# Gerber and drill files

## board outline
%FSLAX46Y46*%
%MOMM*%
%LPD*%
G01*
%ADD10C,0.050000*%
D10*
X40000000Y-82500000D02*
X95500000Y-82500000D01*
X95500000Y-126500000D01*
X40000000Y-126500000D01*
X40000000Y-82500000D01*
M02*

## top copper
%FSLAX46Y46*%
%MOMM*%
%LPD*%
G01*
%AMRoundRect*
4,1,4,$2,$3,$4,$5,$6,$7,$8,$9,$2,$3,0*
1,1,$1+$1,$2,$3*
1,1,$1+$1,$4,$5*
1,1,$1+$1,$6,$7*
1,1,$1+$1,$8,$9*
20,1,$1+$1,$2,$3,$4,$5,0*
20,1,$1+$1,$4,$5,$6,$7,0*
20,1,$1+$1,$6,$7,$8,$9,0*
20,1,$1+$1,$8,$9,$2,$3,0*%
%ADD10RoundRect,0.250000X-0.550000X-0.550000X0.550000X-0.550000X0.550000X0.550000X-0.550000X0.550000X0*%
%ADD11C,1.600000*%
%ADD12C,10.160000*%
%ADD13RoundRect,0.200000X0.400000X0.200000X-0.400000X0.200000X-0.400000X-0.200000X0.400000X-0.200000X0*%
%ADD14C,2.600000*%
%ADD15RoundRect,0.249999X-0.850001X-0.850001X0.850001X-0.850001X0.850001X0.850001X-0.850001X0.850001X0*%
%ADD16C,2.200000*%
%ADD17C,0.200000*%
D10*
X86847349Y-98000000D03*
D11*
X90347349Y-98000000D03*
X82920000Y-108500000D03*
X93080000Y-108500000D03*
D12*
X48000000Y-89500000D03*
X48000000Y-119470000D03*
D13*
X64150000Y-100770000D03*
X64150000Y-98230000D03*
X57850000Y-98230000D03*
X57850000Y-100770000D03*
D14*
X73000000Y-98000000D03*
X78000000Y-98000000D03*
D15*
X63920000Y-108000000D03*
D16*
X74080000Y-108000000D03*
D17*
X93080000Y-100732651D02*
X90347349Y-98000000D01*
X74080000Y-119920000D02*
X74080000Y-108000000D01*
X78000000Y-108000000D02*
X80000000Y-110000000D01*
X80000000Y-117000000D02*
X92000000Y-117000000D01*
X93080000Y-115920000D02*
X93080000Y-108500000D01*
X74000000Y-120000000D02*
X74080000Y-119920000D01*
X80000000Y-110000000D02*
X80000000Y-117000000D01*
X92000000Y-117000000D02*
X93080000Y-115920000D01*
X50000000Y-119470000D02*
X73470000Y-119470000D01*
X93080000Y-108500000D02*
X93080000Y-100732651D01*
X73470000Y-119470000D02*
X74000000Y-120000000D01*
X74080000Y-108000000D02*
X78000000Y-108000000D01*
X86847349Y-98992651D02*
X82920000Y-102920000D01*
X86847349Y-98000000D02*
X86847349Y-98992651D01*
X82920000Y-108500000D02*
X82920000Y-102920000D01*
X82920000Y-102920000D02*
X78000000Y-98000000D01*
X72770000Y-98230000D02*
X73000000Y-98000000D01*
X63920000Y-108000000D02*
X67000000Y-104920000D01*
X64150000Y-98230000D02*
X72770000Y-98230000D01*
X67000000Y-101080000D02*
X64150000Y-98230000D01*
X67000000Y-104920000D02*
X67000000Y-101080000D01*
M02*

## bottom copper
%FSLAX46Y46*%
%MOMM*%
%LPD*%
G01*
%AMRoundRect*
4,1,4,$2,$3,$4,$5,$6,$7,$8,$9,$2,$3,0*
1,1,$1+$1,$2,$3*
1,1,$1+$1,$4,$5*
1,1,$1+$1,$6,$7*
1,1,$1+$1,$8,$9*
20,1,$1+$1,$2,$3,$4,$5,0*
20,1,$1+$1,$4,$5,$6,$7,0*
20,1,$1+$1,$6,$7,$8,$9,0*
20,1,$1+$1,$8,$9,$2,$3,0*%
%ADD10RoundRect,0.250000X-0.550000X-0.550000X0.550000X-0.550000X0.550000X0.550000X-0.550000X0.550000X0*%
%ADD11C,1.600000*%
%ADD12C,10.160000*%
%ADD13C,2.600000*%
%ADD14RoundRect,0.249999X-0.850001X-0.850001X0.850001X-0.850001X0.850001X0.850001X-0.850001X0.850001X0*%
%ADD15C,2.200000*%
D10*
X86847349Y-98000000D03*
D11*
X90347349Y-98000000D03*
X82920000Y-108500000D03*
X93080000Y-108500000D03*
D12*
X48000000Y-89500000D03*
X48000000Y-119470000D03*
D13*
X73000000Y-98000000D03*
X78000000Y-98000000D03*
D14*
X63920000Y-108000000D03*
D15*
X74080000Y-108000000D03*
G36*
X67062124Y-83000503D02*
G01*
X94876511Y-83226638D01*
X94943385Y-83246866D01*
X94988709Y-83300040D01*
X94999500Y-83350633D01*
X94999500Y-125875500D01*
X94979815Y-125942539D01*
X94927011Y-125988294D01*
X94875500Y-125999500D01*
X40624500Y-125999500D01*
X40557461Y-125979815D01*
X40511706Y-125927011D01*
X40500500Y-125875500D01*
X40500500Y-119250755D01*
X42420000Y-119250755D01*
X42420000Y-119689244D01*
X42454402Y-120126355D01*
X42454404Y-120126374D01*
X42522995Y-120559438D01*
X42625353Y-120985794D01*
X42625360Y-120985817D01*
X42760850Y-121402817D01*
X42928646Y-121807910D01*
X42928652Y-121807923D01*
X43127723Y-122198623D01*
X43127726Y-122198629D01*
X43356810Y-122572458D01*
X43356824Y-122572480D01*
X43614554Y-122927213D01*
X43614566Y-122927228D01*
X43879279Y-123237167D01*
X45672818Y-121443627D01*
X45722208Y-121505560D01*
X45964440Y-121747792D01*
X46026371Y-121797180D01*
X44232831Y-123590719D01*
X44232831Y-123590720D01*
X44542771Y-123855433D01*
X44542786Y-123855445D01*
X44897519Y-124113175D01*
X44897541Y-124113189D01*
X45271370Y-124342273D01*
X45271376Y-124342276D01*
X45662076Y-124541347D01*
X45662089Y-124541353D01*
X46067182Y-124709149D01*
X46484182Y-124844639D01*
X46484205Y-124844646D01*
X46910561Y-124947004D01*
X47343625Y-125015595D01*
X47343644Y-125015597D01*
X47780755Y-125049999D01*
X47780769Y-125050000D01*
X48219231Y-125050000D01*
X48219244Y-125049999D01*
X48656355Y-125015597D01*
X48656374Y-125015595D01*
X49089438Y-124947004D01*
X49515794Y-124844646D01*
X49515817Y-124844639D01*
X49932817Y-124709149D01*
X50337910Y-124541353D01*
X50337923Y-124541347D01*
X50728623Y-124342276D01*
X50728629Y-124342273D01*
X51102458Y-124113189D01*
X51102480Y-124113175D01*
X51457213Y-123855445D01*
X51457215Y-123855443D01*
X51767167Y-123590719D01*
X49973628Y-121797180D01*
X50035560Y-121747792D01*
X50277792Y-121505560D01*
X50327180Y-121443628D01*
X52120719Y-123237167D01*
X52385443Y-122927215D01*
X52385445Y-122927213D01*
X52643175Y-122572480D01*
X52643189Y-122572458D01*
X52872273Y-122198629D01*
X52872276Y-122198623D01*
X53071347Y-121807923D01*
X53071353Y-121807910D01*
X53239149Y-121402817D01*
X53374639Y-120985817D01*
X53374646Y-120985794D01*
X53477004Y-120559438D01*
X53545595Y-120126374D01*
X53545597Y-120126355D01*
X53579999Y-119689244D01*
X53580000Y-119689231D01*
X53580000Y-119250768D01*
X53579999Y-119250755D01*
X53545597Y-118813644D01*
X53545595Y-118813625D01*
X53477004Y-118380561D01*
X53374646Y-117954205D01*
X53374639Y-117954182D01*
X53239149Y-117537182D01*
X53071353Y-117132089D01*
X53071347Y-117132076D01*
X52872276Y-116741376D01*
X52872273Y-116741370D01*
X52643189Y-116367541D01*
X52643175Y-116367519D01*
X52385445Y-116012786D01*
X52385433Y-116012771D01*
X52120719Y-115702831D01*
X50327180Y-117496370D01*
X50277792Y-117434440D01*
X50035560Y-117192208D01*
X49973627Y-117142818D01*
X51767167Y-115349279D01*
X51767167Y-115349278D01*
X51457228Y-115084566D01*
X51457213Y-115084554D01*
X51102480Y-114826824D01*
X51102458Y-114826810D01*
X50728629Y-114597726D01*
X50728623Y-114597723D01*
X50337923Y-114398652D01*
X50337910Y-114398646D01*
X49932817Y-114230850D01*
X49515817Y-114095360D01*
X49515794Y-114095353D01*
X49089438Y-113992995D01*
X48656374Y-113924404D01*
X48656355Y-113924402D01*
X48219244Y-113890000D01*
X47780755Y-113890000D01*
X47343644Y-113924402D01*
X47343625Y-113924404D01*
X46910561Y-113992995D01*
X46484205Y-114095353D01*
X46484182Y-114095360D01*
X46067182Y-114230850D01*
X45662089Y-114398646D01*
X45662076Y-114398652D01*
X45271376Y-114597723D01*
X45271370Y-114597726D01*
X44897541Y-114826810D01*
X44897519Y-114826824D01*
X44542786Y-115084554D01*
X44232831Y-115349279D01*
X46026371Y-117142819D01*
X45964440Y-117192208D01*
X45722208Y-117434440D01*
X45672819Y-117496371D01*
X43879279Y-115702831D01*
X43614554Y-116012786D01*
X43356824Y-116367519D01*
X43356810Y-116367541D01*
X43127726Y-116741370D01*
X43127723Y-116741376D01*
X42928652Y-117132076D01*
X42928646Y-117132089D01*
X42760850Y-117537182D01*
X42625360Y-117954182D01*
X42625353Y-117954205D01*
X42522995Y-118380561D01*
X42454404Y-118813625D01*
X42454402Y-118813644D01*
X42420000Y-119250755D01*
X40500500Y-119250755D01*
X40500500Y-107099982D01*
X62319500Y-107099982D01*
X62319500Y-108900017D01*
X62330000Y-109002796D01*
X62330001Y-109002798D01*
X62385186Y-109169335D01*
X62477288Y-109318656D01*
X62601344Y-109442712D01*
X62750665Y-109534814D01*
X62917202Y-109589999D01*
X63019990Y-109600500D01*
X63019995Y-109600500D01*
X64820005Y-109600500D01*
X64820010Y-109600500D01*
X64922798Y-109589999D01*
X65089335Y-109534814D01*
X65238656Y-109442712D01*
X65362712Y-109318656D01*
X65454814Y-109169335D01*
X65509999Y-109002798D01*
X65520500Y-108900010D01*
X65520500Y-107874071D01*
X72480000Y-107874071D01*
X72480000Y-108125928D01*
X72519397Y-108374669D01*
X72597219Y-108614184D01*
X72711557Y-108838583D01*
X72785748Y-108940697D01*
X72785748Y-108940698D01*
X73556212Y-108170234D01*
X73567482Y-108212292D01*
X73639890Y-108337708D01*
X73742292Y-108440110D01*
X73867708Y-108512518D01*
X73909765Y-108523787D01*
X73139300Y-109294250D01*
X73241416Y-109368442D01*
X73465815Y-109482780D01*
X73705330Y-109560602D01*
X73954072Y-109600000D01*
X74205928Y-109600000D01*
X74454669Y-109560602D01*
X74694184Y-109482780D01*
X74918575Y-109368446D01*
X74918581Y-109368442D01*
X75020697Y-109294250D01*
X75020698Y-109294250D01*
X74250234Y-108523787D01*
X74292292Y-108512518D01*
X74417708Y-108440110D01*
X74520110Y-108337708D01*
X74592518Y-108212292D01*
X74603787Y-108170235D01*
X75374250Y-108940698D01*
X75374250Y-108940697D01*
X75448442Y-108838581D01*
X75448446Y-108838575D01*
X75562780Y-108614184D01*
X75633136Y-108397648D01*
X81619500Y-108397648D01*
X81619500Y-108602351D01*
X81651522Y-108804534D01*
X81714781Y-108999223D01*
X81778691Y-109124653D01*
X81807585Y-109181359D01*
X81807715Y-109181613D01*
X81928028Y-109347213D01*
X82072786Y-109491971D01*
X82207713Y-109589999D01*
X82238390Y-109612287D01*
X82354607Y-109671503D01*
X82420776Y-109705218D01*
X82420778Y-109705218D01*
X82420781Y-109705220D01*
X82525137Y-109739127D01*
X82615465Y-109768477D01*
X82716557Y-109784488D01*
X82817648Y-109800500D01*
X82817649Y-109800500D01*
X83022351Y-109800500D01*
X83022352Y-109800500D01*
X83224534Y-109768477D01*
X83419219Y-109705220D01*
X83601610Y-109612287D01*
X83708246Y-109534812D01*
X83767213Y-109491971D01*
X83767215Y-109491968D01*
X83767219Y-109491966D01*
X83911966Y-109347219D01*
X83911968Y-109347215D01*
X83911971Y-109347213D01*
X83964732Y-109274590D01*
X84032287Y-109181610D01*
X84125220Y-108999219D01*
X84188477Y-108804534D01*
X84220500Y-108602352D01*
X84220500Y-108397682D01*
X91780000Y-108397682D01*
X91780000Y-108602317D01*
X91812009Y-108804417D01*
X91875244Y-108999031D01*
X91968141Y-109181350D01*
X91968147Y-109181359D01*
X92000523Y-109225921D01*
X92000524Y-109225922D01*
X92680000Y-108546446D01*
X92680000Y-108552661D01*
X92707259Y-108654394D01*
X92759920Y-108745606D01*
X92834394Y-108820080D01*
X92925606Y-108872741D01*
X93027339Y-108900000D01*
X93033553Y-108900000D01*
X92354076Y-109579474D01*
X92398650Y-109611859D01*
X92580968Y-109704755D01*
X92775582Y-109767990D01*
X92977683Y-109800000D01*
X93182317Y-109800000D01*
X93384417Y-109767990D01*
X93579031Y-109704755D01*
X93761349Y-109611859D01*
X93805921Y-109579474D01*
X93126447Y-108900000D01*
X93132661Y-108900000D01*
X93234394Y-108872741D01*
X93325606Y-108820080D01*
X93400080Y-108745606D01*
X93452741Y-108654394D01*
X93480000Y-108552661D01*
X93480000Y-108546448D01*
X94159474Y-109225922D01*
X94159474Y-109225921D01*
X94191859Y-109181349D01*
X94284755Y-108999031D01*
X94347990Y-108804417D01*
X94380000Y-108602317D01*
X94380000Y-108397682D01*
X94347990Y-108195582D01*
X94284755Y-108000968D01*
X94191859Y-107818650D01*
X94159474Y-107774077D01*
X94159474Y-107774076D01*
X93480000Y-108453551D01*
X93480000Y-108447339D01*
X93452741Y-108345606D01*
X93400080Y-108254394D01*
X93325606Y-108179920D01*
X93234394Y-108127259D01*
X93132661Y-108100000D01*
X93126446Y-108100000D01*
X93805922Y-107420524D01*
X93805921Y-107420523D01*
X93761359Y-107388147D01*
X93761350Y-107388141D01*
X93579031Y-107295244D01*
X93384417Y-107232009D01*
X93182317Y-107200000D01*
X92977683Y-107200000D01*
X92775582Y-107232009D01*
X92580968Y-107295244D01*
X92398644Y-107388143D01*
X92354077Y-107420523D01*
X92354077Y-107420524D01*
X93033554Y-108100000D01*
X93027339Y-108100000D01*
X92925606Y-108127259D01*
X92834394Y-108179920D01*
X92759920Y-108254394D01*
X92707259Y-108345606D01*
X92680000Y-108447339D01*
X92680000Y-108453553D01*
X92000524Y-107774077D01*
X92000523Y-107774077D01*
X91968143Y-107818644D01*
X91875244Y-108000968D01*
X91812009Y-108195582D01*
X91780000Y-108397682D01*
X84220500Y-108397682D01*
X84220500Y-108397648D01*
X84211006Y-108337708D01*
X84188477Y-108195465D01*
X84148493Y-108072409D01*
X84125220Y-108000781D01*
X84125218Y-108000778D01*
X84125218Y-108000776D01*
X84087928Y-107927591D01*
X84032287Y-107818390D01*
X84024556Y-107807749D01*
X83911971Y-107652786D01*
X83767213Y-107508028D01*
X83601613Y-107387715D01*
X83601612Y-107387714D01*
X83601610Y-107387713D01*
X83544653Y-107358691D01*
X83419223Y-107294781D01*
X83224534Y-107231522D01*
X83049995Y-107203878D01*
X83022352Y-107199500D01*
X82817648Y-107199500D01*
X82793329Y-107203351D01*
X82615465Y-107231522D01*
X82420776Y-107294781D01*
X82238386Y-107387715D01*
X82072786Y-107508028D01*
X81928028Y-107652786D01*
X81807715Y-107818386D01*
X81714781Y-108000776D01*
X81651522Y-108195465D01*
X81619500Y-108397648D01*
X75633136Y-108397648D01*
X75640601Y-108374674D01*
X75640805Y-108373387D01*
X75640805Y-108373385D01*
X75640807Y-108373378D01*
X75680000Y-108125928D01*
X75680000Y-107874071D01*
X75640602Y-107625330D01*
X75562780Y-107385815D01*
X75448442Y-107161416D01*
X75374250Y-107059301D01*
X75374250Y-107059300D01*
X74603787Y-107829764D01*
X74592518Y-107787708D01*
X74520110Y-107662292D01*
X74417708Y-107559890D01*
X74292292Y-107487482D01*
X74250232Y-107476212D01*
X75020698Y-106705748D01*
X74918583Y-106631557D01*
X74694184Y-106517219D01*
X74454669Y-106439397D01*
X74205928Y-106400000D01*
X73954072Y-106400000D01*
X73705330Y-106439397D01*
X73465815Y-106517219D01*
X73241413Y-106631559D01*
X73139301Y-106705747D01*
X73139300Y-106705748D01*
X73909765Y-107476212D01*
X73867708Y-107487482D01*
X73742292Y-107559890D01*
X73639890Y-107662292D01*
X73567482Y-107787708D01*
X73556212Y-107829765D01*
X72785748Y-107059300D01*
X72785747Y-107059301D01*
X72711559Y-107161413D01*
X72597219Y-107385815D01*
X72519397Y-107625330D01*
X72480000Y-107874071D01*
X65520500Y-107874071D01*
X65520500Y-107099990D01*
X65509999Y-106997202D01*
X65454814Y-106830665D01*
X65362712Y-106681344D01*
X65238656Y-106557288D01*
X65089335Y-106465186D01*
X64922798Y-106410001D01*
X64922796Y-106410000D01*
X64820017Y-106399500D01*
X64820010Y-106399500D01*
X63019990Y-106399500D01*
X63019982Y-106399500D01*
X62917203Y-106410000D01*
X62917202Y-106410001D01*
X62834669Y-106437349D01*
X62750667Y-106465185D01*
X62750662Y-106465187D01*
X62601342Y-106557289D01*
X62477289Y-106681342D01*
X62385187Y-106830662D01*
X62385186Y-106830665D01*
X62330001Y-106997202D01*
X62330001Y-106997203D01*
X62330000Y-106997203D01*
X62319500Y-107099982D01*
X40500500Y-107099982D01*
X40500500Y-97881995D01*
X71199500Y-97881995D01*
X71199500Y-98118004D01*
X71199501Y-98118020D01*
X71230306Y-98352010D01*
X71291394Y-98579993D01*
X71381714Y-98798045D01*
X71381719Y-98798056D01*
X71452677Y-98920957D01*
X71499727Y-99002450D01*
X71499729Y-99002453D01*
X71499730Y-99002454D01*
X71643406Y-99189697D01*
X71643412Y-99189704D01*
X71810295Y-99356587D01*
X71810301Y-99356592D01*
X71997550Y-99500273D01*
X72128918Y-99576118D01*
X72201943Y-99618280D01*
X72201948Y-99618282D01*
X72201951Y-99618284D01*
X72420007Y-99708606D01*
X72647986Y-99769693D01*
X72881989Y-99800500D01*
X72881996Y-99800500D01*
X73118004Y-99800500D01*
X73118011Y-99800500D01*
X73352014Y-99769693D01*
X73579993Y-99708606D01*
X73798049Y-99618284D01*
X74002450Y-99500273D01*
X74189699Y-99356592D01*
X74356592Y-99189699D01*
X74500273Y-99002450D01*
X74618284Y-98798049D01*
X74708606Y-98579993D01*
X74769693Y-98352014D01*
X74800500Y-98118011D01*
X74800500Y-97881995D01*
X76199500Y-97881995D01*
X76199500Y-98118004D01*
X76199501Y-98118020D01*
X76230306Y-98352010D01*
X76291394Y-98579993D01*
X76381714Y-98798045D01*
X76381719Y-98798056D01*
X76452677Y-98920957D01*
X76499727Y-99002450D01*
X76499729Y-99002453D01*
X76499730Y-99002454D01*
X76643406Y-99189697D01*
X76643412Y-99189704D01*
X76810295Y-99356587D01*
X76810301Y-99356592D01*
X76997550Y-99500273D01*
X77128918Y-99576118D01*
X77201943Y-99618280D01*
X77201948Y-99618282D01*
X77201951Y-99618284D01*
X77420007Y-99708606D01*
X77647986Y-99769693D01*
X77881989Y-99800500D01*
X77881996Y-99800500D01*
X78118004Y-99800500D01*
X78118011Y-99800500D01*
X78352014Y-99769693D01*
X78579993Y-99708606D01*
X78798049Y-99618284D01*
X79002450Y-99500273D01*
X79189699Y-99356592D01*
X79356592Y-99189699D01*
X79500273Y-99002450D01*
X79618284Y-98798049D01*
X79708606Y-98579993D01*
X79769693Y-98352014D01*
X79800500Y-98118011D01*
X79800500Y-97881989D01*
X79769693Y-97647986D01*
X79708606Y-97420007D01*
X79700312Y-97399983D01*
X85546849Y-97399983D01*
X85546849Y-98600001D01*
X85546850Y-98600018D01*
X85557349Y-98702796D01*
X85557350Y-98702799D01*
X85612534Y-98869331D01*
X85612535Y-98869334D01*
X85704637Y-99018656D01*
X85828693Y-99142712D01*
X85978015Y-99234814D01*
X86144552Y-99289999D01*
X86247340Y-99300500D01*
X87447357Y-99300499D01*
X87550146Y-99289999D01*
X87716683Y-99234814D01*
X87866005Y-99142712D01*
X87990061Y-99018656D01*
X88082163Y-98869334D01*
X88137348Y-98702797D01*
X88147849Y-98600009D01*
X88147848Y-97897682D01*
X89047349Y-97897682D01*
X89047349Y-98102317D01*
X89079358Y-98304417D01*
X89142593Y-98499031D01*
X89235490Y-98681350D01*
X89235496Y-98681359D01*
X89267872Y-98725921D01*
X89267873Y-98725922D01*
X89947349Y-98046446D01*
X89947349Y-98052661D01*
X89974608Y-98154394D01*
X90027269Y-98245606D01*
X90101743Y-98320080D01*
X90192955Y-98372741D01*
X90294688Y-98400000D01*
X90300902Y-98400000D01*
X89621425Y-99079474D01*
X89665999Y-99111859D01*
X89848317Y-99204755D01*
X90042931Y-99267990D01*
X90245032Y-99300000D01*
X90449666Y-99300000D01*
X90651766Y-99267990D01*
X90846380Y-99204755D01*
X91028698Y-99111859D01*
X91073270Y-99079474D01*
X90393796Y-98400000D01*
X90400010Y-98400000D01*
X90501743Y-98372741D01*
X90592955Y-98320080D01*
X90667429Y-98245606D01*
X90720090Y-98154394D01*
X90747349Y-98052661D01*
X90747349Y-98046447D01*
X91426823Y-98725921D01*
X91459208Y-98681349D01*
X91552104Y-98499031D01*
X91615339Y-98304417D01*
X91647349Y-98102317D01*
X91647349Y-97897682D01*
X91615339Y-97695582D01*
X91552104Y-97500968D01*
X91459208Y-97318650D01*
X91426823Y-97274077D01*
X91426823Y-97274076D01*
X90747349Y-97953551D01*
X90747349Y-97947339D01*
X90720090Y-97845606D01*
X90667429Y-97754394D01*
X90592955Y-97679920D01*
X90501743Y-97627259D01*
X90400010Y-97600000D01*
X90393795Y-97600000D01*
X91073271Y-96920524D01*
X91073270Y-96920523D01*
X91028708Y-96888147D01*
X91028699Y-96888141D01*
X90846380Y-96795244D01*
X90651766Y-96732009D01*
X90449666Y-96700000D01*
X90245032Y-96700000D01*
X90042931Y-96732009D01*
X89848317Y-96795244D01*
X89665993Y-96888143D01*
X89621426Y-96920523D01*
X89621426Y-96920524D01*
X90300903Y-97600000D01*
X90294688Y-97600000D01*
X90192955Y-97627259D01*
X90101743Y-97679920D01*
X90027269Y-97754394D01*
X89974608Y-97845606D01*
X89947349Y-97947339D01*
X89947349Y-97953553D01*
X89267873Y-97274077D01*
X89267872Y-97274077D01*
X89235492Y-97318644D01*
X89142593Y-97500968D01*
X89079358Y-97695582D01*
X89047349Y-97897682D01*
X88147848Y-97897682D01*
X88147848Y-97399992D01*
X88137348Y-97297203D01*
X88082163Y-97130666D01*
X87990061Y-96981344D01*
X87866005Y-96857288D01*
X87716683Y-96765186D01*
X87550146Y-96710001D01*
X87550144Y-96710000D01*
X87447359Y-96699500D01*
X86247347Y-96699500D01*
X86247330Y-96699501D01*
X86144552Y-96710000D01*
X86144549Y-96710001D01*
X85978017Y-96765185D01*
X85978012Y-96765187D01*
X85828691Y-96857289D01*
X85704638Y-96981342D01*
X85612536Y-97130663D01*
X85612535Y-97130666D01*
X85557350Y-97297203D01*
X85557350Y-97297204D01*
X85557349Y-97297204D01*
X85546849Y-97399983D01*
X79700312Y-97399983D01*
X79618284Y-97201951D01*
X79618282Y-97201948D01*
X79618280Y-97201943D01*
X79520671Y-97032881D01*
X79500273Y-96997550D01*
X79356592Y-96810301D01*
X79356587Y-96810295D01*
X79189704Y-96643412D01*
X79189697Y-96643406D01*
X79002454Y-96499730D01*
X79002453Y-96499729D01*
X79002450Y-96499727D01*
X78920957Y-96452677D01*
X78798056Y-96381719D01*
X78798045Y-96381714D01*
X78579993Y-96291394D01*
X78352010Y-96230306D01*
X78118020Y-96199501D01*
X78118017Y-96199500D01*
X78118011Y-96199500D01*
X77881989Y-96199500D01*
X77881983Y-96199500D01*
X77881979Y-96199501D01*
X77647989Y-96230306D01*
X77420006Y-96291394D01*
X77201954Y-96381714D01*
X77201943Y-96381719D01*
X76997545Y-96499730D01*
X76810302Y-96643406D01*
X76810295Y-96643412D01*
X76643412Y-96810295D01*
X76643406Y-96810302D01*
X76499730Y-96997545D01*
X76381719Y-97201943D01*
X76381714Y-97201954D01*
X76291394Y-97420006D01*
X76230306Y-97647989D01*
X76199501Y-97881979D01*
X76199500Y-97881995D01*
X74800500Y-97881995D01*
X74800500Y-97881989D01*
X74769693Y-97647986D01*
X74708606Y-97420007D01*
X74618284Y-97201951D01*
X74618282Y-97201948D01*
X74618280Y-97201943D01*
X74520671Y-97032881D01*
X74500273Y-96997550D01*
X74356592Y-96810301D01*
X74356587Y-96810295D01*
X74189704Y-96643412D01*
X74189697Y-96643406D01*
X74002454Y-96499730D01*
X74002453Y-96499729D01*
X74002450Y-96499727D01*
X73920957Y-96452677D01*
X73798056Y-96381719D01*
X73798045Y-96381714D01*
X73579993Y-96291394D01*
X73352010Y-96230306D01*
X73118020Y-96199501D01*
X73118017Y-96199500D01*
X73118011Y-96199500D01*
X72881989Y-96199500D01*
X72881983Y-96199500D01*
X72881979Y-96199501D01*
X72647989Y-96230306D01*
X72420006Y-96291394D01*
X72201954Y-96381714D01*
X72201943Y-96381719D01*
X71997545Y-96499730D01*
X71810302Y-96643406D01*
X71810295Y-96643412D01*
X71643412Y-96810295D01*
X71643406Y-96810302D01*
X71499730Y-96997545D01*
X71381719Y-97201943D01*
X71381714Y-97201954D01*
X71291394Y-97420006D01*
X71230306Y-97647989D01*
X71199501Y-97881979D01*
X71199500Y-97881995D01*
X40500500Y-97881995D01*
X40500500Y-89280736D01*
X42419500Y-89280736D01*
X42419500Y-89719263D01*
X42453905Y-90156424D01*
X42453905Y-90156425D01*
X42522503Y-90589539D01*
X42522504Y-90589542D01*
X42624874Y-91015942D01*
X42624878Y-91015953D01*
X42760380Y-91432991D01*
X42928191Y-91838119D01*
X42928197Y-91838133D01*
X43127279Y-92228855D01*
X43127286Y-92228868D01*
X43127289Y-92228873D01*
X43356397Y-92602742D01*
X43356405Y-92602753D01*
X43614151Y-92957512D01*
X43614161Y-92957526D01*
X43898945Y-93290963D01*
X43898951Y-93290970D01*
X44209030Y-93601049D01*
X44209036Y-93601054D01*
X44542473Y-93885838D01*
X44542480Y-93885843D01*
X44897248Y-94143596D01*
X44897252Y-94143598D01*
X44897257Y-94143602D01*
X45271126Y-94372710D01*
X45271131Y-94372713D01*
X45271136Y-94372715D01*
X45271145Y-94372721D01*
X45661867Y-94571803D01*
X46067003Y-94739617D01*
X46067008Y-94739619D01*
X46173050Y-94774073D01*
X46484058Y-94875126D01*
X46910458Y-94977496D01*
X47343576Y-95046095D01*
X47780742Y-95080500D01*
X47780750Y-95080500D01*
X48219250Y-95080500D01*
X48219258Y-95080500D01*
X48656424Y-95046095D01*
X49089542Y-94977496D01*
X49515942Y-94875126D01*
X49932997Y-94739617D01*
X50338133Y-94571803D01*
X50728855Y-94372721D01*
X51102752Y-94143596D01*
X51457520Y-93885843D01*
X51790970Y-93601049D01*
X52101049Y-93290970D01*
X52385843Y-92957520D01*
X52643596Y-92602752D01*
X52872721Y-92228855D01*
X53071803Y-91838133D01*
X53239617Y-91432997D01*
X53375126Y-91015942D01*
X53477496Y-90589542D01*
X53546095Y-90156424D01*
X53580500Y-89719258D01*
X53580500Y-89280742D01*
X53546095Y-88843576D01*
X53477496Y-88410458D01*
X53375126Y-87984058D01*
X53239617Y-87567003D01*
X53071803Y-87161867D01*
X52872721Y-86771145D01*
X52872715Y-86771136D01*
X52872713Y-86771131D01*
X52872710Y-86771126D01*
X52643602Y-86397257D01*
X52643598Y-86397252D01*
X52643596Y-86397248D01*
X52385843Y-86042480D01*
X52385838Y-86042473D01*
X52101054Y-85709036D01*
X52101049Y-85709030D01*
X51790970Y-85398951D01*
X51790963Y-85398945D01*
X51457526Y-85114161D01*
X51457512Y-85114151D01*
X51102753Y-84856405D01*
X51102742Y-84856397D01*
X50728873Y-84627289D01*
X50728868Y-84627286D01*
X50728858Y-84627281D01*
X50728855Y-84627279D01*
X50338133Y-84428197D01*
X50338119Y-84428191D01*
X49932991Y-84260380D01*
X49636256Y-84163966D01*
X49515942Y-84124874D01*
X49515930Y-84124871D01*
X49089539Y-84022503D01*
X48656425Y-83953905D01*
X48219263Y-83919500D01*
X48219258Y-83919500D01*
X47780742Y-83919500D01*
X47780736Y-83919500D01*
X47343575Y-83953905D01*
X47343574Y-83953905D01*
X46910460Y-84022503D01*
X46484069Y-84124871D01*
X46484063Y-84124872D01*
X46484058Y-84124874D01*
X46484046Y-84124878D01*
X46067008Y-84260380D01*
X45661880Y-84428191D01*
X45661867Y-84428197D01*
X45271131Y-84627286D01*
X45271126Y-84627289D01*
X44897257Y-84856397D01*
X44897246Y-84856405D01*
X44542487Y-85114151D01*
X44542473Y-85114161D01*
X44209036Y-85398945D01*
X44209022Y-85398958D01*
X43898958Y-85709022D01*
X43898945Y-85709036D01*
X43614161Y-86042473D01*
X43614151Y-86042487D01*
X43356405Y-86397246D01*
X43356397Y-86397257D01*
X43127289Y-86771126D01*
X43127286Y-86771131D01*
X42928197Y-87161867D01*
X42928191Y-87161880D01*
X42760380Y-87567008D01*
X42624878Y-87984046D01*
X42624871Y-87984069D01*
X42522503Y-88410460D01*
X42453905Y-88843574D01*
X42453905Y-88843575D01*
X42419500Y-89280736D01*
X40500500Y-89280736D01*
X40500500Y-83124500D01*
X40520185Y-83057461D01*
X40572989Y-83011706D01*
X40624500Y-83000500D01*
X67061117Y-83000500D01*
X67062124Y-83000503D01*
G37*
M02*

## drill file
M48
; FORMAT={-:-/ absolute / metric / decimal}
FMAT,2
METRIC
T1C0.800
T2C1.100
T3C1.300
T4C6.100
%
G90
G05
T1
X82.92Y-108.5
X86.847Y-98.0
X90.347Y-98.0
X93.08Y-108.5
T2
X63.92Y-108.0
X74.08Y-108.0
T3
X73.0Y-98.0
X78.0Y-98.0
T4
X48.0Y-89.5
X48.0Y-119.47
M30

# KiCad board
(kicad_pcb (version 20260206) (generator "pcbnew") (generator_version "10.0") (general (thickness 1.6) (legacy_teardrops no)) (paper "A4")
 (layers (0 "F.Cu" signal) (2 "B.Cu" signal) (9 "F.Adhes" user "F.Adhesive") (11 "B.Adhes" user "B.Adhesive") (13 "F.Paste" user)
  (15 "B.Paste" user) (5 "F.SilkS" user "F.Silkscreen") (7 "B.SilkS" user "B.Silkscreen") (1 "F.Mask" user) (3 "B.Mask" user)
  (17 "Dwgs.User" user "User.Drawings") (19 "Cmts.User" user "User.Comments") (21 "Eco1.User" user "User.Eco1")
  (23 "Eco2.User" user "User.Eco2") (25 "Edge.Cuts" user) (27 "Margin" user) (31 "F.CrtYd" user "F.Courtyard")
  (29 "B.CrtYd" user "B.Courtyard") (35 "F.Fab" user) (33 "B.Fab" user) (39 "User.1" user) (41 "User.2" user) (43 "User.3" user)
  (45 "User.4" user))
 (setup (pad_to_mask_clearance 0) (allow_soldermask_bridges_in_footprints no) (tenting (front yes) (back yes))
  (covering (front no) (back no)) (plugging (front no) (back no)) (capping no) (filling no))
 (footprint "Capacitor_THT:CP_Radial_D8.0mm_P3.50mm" (layer "F.Cu") (at 86.847349 98)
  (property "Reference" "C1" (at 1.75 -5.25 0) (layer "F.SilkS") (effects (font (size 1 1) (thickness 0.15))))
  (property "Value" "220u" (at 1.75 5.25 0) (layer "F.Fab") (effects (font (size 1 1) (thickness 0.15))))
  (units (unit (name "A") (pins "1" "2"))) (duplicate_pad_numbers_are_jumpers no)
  (pad "1" thru_hole roundrect (at 0 0) (size 1.6 1.6) (drill 0.8) (layers "*.Cu" "*.Mask") (remove_unused_layers no)
   (roundrect_rratio 0.15625) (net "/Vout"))
  (pad "2" thru_hole circle (at 3.5 0) (size 1.6 1.6) (drill 0.8) (layers "*.Cu" "*.Mask") (remove_unused_layers no) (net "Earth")))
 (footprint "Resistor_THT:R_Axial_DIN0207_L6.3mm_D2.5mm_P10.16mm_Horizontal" (layer "F.Cu") (at 82.92 108.5)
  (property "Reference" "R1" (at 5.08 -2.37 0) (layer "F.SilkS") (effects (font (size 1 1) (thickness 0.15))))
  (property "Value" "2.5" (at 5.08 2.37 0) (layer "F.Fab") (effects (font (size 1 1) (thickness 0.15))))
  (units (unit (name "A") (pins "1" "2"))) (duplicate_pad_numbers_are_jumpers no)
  (pad "1" thru_hole circle (at 0 0) (size 1.6 1.6) (drill 0.8) (layers "*.Cu" "*.Mask") (remove_unused_layers no) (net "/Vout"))
  (pad "2" thru_hole circle (at 10.16 0) (size 1.6 1.6) (drill 0.8) (layers "*.Cu" "*.Mask") (remove_unused_layers no) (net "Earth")))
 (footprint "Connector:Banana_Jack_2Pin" (layer "F.Cu") (at 48 89.5 -90)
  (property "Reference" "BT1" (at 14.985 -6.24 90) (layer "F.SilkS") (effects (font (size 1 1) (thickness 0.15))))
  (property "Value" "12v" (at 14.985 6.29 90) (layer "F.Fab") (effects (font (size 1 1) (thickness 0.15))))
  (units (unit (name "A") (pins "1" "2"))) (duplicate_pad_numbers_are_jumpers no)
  (pad "1" thru_hole circle (at 0 0 270) (size 10.16 10.16) (drill 6.1) (layers "*.Cu" "*.Mask") (remove_unused_layers no) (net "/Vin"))
  (pad "2" thru_hole circle (at 29.97 0 270) (size 10.16 10.16) (drill 6.1) (layers "*.Cu" "*.Mask") (remove_unused_layers no) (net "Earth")))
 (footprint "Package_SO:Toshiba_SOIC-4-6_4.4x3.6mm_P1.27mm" (layer "F.Cu") (at 61 99.5 180)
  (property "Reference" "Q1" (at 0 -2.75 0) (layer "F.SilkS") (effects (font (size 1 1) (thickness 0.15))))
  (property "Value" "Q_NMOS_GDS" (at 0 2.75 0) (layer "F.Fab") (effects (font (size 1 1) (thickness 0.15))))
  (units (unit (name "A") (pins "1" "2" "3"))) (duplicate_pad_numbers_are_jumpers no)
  (pad "1" smd roundrect (at -3.15 -1.27 180) (size 1.2 0.8) (layers "F.Cu" "F.Mask" "F.Paste") (roundrect_rratio 0.25)
   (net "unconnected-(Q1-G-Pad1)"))
  (pad "3" smd roundrect (at -3.15 1.27 180) (size 1.2 0.8) (layers "F.Cu" "F.Mask" "F.Paste") (roundrect_rratio 0.25) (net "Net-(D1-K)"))
  (pad "4" smd roundrect (at 3.15 1.27 180) (size 1.2 0.8) (layers "F.Cu" "F.Mask" "F.Paste") (roundrect_rratio 0.25))
  (pad "6" smd roundrect (at 3.15 -1.27 180) (size 1.2 0.8) (layers "F.Cu" "F.Mask" "F.Paste") (roundrect_rratio 0.25)))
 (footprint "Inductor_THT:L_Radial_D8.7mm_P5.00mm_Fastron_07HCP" (layer "F.Cu") (at 73 98)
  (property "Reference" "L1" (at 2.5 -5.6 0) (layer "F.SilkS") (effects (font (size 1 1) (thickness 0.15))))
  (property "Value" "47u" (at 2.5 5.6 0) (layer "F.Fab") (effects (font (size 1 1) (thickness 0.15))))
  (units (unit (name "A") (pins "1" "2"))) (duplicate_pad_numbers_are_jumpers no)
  (pad "1" thru_hole circle (at 0 0) (size 2.6 2.6) (drill 1.3) (layers "*.Cu" "*.Mask") (remove_unused_layers no) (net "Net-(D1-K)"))
  (pad "2" thru_hole circle (at 5 0) (size 2.6 2.6) (drill 1.3) (layers "*.Cu" "*.Mask") (remove_unused_layers no) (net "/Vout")))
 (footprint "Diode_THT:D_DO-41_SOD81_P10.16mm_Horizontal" (layer "F.Cu") (at 63.92 108)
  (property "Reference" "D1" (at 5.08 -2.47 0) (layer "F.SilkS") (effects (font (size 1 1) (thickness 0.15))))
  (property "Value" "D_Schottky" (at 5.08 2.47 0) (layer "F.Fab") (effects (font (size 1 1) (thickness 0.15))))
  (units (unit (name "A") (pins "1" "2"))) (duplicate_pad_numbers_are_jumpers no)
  (pad "1" thru_hole roundrect (at 0 0) (size 2.2 2.2) (drill 1.1) (layers "*.Cu" "*.Mask") (remove_unused_layers no)
   (roundrect_rratio 0.113636) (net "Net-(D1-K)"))
  (pad "2" thru_hole circle (at 10.16 0) (size 2.2 2.2) (drill 1.1) (layers "*.Cu" "*.Mask") (remove_unused_layers no) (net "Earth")))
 (gr_rect (start 40 82.5) (end 95.5 126.5) (stroke (width 0.05) (type default)) (fill no) (layer "Edge.Cuts"))
 (segment (start 93.08 100.732651) (end 90.347349 98) (width 0.2) (layer "F.Cu") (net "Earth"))
 (segment (start 74.08 119.92) (end 74.08 108) (width 0.2) (layer "F.Cu") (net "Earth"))
 (segment (start 78 108) (end 80 110) (width 0.2) (layer "F.Cu") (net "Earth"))
 (segment (start 80 117) (end 92 117) (width 0.2) (layer "F.Cu") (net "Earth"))
 (segment (start 93.08 115.92) (end 93.08 108.5) (width 0.2) (layer "F.Cu") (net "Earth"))
 (segment (start 74 120) (end 74.08 119.92) (width 0.2) (layer "F.Cu") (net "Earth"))
 (segment (start 80 110) (end 80 117) (width 0.2) (layer "F.Cu") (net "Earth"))
 (segment (start 92 117) (end 93.08 115.92) (width 0.2) (layer "F.Cu") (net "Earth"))
 (segment (start 50 119.47) (end 73.47 119.47) (width 0.2) (layer "F.Cu") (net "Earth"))
 (segment (start 93.08 108.5) (end 93.08 100.732651) (width 0.2) (layer "F.Cu") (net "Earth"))
 (segment (start 73.47 119.47) (end 74 120) (width 0.2) (layer "F.Cu") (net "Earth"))
 (segment (start 74.08 108) (end 78 108) (width 0.2) (layer "F.Cu") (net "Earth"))
 (segment (start 86.847349 98.992651) (end 82.92 102.92) (width 0.2) (layer "F.Cu") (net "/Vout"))
 (segment (start 86.847349 98) (end 86.847349 98.992651) (width 0.2) (layer "F.Cu") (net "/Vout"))
 (segment (start 82.92 108.5) (end 82.92 102.92) (width 0.2) (layer "F.Cu") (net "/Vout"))
 (segment (start 82.92 102.92) (end 78 98) (width 0.2) (layer "F.Cu") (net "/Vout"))
 (segment (start 72.77 98.23) (end 73 98) (width 0.2) (layer "F.Cu") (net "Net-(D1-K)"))
 (segment (start 63.92 108) (end 67 104.92) (width 0.2) (layer "F.Cu") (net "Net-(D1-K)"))
 (segment (start 64.15 98.23) (end 72.77 98.23) (width 0.2) (layer "F.Cu") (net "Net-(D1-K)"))
 (segment (start 67 101.08) (end 64.15 98.23) (width 0.2) (layer "F.Cu") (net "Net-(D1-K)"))
 (segment (start 67 104.92) (end 67 101.08) (width 0.2) (layer "F.Cu") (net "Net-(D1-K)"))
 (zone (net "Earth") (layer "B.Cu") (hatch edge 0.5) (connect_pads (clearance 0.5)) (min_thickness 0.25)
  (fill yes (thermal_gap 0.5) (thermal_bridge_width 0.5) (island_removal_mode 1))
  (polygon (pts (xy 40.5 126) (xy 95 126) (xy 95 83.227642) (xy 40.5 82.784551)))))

